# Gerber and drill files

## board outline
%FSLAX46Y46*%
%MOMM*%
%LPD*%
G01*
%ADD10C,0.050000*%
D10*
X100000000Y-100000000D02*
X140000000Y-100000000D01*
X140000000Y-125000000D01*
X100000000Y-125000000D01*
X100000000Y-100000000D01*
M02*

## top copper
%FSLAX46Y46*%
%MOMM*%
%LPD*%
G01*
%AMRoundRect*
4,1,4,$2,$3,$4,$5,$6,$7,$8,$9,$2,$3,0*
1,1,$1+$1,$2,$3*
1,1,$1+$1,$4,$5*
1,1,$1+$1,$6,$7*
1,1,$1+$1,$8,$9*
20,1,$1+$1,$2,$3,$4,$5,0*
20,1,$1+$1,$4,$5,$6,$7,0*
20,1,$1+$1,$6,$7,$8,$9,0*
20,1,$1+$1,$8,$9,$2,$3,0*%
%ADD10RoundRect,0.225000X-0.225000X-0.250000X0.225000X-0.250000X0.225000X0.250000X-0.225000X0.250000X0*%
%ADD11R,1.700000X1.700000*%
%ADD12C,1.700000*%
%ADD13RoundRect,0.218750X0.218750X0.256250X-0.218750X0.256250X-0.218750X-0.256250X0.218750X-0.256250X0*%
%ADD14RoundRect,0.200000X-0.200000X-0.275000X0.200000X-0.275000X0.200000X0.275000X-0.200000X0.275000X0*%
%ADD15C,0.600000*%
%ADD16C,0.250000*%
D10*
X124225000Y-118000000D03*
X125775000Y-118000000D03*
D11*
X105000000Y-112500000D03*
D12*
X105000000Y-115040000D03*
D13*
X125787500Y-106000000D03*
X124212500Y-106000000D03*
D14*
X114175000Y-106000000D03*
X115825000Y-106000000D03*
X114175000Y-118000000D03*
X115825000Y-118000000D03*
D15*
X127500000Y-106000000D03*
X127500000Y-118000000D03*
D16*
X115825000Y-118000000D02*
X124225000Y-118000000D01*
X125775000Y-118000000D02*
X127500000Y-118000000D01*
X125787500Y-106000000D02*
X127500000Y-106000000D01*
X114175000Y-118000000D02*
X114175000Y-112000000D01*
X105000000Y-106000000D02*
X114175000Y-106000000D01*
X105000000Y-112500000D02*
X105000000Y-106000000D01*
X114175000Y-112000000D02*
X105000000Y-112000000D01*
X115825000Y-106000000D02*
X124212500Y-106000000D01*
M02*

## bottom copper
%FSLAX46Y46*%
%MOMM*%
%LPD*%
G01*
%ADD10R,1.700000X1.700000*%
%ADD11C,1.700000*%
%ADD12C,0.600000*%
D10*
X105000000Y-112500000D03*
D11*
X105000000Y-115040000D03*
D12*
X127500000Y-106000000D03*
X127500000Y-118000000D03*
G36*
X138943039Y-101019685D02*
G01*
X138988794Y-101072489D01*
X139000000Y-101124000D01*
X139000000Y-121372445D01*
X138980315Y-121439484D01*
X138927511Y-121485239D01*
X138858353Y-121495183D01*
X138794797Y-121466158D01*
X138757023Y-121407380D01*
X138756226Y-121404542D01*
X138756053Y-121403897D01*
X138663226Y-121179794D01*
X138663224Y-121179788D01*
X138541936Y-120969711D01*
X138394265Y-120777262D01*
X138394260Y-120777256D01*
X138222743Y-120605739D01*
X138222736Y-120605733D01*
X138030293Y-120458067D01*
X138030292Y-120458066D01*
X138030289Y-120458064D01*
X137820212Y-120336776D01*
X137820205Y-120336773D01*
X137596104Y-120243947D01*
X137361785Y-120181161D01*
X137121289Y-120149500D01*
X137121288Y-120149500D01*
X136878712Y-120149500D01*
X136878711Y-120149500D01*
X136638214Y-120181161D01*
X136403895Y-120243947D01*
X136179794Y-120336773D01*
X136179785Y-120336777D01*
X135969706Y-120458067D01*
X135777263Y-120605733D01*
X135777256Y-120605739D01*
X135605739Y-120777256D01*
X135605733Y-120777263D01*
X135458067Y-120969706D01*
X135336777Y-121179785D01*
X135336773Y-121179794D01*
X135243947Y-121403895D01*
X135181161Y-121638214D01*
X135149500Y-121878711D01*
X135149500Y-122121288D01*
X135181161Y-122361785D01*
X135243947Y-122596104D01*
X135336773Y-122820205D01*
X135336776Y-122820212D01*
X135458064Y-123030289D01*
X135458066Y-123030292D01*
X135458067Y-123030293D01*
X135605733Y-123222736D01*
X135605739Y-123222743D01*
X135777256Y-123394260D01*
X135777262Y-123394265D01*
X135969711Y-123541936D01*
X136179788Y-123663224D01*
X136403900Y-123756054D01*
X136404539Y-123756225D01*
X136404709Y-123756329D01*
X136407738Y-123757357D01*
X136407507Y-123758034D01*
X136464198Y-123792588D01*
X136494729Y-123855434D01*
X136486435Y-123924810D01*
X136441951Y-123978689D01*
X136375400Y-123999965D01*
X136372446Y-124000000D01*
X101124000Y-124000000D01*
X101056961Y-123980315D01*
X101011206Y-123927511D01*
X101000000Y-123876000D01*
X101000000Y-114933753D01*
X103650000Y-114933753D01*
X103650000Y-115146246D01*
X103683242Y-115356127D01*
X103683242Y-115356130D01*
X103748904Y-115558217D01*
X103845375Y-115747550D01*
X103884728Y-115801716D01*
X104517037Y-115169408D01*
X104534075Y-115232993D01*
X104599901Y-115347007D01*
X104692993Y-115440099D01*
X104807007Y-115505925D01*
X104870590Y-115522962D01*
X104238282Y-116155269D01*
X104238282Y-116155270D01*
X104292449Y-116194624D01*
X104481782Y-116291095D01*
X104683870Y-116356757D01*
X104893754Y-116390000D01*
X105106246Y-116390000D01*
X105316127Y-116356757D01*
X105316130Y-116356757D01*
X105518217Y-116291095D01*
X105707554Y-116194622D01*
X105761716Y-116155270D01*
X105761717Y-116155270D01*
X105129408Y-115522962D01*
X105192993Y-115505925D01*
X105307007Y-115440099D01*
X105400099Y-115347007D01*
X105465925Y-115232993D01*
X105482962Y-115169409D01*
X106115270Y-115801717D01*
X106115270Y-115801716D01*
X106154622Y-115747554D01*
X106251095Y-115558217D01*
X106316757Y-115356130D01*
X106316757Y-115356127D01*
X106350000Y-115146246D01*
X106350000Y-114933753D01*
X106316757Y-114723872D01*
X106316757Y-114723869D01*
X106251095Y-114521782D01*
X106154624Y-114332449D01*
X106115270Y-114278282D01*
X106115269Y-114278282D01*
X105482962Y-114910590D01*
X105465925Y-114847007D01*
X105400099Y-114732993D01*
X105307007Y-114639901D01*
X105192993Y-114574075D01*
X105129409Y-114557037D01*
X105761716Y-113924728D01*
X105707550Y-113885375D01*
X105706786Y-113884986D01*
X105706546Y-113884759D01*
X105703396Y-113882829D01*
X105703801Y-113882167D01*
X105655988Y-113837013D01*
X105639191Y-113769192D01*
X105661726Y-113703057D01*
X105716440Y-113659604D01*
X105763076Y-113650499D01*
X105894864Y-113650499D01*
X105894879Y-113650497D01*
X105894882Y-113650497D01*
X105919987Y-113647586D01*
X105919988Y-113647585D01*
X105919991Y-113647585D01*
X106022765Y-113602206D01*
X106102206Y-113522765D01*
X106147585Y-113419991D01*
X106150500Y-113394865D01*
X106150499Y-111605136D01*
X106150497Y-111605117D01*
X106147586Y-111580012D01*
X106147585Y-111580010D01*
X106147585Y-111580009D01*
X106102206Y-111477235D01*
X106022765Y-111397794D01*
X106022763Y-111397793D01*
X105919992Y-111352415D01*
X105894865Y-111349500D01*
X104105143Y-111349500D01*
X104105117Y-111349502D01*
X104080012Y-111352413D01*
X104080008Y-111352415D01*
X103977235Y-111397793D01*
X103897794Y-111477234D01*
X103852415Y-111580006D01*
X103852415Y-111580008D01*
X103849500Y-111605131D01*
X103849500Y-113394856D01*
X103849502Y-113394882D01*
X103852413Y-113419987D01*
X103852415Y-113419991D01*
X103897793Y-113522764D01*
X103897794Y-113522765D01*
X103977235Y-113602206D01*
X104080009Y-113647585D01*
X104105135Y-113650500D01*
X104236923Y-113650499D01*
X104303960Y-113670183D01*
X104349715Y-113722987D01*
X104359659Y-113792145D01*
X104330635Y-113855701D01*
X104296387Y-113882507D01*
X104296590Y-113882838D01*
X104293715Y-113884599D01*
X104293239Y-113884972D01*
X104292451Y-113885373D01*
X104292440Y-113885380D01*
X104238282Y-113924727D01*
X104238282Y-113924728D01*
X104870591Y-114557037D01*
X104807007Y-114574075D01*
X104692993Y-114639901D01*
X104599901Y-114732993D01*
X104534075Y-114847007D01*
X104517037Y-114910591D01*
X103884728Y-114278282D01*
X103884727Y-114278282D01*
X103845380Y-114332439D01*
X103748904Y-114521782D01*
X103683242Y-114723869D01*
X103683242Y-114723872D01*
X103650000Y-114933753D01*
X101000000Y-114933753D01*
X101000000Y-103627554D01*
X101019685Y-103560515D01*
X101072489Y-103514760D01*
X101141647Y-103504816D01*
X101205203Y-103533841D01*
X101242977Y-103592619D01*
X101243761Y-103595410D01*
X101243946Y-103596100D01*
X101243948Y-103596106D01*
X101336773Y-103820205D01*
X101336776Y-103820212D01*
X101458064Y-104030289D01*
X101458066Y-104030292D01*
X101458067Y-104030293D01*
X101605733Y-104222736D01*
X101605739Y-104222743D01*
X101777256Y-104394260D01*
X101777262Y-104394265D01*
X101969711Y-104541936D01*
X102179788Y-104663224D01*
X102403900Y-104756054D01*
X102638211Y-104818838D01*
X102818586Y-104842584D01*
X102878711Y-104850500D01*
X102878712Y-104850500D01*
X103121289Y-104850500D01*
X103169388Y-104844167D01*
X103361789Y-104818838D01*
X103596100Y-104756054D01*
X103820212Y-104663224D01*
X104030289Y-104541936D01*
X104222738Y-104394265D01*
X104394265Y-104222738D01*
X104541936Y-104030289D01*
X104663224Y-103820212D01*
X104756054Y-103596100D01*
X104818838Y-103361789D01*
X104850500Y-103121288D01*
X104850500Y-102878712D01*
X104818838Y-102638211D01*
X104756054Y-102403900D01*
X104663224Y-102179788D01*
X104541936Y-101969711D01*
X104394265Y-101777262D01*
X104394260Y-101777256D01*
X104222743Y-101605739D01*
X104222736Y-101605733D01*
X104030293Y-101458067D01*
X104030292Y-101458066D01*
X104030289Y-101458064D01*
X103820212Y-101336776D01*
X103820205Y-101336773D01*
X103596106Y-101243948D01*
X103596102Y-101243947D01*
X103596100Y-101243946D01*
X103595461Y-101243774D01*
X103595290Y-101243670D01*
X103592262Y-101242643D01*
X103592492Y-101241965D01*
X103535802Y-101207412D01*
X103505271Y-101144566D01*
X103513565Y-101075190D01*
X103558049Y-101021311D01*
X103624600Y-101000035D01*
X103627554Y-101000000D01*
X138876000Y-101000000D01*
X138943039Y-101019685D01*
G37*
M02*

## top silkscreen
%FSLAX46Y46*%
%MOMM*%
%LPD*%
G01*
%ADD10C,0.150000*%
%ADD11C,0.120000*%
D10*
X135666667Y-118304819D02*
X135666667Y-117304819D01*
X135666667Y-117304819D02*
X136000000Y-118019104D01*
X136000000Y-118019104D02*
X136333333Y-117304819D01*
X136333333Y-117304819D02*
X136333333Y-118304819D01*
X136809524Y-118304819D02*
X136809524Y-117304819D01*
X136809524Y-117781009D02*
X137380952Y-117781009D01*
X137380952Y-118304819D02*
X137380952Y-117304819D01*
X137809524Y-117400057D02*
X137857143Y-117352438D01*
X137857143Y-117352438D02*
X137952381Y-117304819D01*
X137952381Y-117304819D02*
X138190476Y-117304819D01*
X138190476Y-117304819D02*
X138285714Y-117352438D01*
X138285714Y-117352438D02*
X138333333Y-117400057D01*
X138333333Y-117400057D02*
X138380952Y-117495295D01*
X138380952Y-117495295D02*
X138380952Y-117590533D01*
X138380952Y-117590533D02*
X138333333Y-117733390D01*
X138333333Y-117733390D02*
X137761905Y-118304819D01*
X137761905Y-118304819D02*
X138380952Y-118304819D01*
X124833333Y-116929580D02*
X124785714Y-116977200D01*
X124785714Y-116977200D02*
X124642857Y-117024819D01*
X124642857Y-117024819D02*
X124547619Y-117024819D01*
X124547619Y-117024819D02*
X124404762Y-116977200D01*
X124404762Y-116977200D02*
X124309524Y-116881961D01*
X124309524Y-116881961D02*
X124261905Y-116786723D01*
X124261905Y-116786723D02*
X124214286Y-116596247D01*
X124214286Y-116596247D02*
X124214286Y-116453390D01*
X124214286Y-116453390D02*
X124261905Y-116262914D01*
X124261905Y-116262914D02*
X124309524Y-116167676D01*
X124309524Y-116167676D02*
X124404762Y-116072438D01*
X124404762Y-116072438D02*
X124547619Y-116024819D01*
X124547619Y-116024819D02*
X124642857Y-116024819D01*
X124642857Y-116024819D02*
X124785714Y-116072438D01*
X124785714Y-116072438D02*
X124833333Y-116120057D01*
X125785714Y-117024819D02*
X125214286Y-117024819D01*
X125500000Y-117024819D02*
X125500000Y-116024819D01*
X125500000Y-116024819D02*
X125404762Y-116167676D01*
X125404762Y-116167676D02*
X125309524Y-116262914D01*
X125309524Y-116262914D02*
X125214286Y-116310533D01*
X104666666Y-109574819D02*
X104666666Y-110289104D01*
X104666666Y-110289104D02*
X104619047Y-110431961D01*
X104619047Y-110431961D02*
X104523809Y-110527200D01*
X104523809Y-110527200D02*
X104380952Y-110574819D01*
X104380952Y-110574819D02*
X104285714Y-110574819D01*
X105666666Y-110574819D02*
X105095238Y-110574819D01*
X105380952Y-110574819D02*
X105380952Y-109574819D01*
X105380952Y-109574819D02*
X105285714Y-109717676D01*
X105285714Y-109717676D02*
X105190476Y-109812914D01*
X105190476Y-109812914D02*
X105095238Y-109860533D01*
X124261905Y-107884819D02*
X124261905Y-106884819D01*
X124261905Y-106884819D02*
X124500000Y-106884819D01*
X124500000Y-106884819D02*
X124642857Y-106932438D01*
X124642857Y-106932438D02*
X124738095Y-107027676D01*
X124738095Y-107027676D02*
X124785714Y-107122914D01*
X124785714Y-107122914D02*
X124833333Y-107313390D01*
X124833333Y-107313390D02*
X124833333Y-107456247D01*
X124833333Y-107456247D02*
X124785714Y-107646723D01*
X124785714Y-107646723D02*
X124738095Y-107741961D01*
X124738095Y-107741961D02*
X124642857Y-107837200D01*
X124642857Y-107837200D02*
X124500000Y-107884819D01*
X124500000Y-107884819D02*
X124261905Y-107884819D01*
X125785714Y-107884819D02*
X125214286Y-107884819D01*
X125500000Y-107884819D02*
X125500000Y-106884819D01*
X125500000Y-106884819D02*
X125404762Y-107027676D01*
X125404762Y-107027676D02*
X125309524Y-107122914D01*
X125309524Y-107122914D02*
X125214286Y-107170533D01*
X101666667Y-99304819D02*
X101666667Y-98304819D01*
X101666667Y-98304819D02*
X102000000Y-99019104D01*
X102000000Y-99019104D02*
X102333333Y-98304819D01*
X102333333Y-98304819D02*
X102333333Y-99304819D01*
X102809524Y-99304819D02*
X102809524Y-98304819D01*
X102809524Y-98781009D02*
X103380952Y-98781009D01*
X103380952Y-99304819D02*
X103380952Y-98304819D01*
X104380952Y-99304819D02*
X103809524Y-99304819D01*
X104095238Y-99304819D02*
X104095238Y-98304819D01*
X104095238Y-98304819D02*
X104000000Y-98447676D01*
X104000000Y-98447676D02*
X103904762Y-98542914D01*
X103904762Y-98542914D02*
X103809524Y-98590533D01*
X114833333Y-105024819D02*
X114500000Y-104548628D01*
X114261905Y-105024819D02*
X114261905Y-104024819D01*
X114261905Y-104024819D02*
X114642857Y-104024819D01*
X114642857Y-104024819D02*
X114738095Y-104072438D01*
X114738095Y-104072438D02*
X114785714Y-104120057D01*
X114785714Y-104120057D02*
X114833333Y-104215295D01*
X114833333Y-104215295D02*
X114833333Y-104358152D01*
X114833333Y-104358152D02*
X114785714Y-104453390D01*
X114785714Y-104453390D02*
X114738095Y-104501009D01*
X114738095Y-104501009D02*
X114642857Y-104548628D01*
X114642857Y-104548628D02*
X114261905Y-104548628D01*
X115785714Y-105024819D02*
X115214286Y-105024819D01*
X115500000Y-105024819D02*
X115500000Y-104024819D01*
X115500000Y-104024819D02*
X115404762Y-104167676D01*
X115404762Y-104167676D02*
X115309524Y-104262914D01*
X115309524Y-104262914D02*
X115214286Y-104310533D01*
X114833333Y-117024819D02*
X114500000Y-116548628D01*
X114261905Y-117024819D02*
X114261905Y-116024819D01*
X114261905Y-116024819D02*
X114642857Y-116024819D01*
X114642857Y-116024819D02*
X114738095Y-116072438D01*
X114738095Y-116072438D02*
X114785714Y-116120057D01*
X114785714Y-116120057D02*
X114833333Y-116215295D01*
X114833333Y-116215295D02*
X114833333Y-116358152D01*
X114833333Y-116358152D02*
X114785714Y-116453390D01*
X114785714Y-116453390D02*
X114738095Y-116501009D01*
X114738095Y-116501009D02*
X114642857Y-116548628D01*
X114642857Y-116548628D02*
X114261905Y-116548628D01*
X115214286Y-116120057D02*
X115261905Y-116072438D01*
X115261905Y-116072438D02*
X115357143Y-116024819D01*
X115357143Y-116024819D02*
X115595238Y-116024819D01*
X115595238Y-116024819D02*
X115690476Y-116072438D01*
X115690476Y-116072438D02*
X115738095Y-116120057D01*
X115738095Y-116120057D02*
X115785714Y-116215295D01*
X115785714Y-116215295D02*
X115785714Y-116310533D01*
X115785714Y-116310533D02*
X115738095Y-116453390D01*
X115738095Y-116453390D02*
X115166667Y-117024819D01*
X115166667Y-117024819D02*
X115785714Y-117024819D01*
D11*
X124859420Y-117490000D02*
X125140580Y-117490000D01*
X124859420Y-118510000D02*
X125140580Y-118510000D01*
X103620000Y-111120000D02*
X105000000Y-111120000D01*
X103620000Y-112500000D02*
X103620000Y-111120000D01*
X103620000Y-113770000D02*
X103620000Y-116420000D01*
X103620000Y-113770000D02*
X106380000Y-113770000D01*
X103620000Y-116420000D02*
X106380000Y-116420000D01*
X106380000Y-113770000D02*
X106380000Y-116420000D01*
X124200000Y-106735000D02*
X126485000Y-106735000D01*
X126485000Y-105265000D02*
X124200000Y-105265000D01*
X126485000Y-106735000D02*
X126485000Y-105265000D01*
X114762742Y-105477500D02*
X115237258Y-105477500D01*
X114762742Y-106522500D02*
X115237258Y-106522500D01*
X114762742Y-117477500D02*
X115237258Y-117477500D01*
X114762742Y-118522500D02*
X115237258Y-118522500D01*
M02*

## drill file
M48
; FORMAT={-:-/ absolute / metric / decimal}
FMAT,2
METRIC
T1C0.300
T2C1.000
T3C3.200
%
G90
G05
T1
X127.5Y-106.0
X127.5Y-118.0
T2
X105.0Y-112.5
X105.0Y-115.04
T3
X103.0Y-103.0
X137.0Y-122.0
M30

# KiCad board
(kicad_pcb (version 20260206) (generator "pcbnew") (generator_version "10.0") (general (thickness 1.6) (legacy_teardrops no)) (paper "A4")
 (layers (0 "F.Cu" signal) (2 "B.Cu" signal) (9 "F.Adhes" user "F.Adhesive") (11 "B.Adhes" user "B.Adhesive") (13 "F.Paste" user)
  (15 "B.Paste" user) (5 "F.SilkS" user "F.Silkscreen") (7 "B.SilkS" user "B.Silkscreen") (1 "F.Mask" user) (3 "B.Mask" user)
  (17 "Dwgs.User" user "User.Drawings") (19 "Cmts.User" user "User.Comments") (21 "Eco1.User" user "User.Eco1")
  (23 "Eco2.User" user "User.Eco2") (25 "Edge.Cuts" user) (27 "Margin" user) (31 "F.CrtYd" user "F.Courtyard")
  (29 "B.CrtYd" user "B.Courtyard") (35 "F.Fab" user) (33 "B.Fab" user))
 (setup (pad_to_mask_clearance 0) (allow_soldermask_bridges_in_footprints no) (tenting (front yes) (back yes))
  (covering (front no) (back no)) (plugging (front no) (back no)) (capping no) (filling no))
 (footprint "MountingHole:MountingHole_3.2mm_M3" (layer "F.Cu") (at 137 122)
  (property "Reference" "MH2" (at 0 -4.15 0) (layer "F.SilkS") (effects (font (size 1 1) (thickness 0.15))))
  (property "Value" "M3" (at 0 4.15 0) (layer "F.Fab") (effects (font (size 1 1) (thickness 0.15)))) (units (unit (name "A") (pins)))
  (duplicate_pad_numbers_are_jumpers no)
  (pad "" np_thru_hole circle (at 0 0) (size 3.2 3.2) (drill 3.2) (layers "*.Cu" "*.Mask")))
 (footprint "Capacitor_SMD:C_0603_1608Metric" (layer "F.Cu") (at 125 118)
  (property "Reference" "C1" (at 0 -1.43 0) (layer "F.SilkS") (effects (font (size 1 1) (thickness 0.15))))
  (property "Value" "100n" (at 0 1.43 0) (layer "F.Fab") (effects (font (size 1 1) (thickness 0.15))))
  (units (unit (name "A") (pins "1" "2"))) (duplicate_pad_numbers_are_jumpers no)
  (fp_line (start -0.14058 -0.51) (end 0.14058 -0.51) (stroke (width 0.12) (type solid)) (layer "F.SilkS"))
  (fp_line (start -0.14058 0.51) (end 0.14058 0.51) (stroke (width 0.12) (type solid)) (layer "F.SilkS"))
  (pad "1" smd roundrect (at -0.775 0) (size 0.9 0.95) (layers "F.Cu" "F.Mask" "F.Paste") (roundrect_rratio 0.25) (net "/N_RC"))
  (pad "2" smd roundrect (at 0.775 0) (size 0.9 0.95) (layers "F.Cu" "F.Mask" "F.Paste") (roundrect_rratio 0.25) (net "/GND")))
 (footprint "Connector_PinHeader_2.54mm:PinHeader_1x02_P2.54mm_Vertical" (layer "F.Cu") (at 105 112.5)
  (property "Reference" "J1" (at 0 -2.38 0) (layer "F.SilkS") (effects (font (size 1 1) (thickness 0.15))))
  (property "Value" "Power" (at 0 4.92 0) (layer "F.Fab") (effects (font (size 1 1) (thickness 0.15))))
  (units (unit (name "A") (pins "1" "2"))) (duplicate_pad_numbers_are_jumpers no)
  (fp_line (start -1.38 -1.38) (end 0 -1.38) (stroke (width 0.12) (type solid)) (layer "F.SilkS"))
  (fp_line (start -1.38 0) (end -1.38 -1.38) (stroke (width 0.12) (type solid)) (layer "F.SilkS"))
  (fp_line (start -1.38 1.27) (end -1.38 3.92) (stroke (width 0.12) (type solid)) (layer "F.SilkS"))
  (fp_line (start -1.38 1.27) (end 1.38 1.27) (stroke (width 0.12) (type solid)) (layer "F.SilkS"))
  (fp_line (start -1.38 3.92) (end 1.38 3.92) (stroke (width 0.12) (type solid)) (layer "F.SilkS"))
  (fp_line (start 1.38 1.27) (end 1.38 3.92) (stroke (width 0.12) (type solid)) (layer "F.SilkS"))
  (pad "1" thru_hole rect (at 0 0) (size 1.7 1.7) (drill 1) (layers "*.Cu" "*.Mask") (remove_unused_layers no) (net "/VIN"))
  (pad "2" thru_hole circle (at 0 2.54) (size 1.7 1.7) (drill 1) (layers "*.Cu" "*.Mask") (remove_unused_layers no) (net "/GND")))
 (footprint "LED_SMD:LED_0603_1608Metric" (layer "F.Cu") (at 125 106 180)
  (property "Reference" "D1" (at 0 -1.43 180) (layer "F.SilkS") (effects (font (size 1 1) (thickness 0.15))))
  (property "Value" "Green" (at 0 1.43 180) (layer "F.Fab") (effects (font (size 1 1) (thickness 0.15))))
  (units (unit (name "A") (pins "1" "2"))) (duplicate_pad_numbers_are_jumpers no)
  (fp_line (start 0.8 -0.735) (end -1.485 -0.735) (stroke (width 0.12) (type solid)) (layer "F.SilkS"))
  (fp_line (start -1.485 0.735) (end 0.8 0.735) (stroke (width 0.12) (type solid)) (layer "F.SilkS"))
  (fp_line (start -1.485 -0.735) (end -1.485 0.735) (stroke (width 0.12) (type solid)) (layer "F.SilkS"))
  (pad "1" smd roundrect (at -0.7875 0 180) (size 0.875 0.95) (layers "F.Cu" "F.Mask" "F.Paste") (roundrect_rratio 0.25) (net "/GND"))
  (pad "2" smd roundrect (at 0.7875 0 180) (size 0.875 0.95) (layers "F.Cu" "F.Mask" "F.Paste") (roundrect_rratio 0.25) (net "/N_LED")))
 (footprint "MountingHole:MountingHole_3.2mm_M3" (layer "F.Cu") (at 103 103)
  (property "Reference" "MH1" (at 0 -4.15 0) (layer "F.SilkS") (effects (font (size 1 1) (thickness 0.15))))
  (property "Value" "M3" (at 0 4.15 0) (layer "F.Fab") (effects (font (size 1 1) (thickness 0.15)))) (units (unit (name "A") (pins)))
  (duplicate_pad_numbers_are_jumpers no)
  (pad "" np_thru_hole circle (at 0 0) (size 3.2 3.2) (drill 3.2) (layers "*.Cu" "*.Mask")))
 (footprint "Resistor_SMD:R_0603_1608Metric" (layer "F.Cu") (at 115 106)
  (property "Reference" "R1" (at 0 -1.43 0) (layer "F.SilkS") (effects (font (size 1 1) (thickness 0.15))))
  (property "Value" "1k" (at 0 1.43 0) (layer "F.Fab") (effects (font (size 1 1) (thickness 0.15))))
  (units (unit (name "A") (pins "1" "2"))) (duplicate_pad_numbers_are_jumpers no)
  (fp_line (start -0.237258 -0.5225) (end 0.237258 -0.5225) (stroke (width 0.12) (type solid)) (layer "F.SilkS"))
  (fp_line (start -0.237258 0.5225) (end 0.237258 0.5225) (stroke (width 0.12) (type solid)) (layer "F.SilkS"))
  (pad "1" smd roundrect (at -0.825 0) (size 0.8 0.95) (layers "F.Cu" "F.Mask" "F.Paste") (roundrect_rratio 0.25) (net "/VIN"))
  (pad "2" smd roundrect (at 0.825 0) (size 0.8 0.95) (layers "F.Cu" "F.Mask" "F.Paste") (roundrect_rratio 0.25) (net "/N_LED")))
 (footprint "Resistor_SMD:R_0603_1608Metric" (layer "F.Cu") (at 115 118)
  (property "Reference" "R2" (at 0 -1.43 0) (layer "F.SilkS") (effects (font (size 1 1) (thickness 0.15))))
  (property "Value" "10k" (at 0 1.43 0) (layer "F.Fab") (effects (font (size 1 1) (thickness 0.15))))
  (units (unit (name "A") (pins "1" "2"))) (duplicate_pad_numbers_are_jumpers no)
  (fp_line (start -0.237258 -0.5225) (end 0.237258 -0.5225) (stroke (width 0.12) (type solid)) (layer "F.SilkS"))
  (fp_line (start -0.237258 0.5225) (end 0.237258 0.5225) (stroke (width 0.12) (type solid)) (layer "F.SilkS"))
  (pad "1" smd roundrect (at -0.825 0) (size 0.8 0.95) (layers "F.Cu" "F.Mask" "F.Paste") (roundrect_rratio 0.25) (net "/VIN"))
  (pad "2" smd roundrect (at 0.825 0) (size 0.8 0.95) (layers "F.Cu" "F.Mask" "F.Paste") (roundrect_rratio 0.25) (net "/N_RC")))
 (gr_rect (start 100 100) (end 140 125) (stroke (width 0.05) (type default)) (fill no) (layer "Edge.Cuts"))
 (segment (start 115.825 118) (end 124.225 118) (width 0.25) (layer "F.Cu") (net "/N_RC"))
 (segment (start 125.775 118) (end 127.5 118) (width 0.25) (layer "F.Cu") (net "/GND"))
 (segment (start 125.7875 106) (end 127.5 106) (width 0.25) (layer "F.Cu") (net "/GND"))
 (via (at 127.5 106) (size 0.6) (drill 0.3) (layers "F.Cu" "B.Cu") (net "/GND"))
 (via (at 127.5 118) (size 0.6) (drill 0.3) (layers "F.Cu" "B.Cu") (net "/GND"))
 (segment (start 114.175 118) (end 114.175 112) (width 0.25) (layer "F.Cu") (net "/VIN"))
 (segment (start 105 106) (end 114.175 106) (width 0.25) (layer "F.Cu") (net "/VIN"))
 (segment (start 105 112.5) (end 105 106) (width 0.25) (layer "F.Cu") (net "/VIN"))
 (segment (start 114.175 112) (end 105 112) (width 0.25) (layer "F.Cu") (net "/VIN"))
 (segment (start 115.825 106) (end 124.2125 106) (width 0.25) (layer "F.Cu") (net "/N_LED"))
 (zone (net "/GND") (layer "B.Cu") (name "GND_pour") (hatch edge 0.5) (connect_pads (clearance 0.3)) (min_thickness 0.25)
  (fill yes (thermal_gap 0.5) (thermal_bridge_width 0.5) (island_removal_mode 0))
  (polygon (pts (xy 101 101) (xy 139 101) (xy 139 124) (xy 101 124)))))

